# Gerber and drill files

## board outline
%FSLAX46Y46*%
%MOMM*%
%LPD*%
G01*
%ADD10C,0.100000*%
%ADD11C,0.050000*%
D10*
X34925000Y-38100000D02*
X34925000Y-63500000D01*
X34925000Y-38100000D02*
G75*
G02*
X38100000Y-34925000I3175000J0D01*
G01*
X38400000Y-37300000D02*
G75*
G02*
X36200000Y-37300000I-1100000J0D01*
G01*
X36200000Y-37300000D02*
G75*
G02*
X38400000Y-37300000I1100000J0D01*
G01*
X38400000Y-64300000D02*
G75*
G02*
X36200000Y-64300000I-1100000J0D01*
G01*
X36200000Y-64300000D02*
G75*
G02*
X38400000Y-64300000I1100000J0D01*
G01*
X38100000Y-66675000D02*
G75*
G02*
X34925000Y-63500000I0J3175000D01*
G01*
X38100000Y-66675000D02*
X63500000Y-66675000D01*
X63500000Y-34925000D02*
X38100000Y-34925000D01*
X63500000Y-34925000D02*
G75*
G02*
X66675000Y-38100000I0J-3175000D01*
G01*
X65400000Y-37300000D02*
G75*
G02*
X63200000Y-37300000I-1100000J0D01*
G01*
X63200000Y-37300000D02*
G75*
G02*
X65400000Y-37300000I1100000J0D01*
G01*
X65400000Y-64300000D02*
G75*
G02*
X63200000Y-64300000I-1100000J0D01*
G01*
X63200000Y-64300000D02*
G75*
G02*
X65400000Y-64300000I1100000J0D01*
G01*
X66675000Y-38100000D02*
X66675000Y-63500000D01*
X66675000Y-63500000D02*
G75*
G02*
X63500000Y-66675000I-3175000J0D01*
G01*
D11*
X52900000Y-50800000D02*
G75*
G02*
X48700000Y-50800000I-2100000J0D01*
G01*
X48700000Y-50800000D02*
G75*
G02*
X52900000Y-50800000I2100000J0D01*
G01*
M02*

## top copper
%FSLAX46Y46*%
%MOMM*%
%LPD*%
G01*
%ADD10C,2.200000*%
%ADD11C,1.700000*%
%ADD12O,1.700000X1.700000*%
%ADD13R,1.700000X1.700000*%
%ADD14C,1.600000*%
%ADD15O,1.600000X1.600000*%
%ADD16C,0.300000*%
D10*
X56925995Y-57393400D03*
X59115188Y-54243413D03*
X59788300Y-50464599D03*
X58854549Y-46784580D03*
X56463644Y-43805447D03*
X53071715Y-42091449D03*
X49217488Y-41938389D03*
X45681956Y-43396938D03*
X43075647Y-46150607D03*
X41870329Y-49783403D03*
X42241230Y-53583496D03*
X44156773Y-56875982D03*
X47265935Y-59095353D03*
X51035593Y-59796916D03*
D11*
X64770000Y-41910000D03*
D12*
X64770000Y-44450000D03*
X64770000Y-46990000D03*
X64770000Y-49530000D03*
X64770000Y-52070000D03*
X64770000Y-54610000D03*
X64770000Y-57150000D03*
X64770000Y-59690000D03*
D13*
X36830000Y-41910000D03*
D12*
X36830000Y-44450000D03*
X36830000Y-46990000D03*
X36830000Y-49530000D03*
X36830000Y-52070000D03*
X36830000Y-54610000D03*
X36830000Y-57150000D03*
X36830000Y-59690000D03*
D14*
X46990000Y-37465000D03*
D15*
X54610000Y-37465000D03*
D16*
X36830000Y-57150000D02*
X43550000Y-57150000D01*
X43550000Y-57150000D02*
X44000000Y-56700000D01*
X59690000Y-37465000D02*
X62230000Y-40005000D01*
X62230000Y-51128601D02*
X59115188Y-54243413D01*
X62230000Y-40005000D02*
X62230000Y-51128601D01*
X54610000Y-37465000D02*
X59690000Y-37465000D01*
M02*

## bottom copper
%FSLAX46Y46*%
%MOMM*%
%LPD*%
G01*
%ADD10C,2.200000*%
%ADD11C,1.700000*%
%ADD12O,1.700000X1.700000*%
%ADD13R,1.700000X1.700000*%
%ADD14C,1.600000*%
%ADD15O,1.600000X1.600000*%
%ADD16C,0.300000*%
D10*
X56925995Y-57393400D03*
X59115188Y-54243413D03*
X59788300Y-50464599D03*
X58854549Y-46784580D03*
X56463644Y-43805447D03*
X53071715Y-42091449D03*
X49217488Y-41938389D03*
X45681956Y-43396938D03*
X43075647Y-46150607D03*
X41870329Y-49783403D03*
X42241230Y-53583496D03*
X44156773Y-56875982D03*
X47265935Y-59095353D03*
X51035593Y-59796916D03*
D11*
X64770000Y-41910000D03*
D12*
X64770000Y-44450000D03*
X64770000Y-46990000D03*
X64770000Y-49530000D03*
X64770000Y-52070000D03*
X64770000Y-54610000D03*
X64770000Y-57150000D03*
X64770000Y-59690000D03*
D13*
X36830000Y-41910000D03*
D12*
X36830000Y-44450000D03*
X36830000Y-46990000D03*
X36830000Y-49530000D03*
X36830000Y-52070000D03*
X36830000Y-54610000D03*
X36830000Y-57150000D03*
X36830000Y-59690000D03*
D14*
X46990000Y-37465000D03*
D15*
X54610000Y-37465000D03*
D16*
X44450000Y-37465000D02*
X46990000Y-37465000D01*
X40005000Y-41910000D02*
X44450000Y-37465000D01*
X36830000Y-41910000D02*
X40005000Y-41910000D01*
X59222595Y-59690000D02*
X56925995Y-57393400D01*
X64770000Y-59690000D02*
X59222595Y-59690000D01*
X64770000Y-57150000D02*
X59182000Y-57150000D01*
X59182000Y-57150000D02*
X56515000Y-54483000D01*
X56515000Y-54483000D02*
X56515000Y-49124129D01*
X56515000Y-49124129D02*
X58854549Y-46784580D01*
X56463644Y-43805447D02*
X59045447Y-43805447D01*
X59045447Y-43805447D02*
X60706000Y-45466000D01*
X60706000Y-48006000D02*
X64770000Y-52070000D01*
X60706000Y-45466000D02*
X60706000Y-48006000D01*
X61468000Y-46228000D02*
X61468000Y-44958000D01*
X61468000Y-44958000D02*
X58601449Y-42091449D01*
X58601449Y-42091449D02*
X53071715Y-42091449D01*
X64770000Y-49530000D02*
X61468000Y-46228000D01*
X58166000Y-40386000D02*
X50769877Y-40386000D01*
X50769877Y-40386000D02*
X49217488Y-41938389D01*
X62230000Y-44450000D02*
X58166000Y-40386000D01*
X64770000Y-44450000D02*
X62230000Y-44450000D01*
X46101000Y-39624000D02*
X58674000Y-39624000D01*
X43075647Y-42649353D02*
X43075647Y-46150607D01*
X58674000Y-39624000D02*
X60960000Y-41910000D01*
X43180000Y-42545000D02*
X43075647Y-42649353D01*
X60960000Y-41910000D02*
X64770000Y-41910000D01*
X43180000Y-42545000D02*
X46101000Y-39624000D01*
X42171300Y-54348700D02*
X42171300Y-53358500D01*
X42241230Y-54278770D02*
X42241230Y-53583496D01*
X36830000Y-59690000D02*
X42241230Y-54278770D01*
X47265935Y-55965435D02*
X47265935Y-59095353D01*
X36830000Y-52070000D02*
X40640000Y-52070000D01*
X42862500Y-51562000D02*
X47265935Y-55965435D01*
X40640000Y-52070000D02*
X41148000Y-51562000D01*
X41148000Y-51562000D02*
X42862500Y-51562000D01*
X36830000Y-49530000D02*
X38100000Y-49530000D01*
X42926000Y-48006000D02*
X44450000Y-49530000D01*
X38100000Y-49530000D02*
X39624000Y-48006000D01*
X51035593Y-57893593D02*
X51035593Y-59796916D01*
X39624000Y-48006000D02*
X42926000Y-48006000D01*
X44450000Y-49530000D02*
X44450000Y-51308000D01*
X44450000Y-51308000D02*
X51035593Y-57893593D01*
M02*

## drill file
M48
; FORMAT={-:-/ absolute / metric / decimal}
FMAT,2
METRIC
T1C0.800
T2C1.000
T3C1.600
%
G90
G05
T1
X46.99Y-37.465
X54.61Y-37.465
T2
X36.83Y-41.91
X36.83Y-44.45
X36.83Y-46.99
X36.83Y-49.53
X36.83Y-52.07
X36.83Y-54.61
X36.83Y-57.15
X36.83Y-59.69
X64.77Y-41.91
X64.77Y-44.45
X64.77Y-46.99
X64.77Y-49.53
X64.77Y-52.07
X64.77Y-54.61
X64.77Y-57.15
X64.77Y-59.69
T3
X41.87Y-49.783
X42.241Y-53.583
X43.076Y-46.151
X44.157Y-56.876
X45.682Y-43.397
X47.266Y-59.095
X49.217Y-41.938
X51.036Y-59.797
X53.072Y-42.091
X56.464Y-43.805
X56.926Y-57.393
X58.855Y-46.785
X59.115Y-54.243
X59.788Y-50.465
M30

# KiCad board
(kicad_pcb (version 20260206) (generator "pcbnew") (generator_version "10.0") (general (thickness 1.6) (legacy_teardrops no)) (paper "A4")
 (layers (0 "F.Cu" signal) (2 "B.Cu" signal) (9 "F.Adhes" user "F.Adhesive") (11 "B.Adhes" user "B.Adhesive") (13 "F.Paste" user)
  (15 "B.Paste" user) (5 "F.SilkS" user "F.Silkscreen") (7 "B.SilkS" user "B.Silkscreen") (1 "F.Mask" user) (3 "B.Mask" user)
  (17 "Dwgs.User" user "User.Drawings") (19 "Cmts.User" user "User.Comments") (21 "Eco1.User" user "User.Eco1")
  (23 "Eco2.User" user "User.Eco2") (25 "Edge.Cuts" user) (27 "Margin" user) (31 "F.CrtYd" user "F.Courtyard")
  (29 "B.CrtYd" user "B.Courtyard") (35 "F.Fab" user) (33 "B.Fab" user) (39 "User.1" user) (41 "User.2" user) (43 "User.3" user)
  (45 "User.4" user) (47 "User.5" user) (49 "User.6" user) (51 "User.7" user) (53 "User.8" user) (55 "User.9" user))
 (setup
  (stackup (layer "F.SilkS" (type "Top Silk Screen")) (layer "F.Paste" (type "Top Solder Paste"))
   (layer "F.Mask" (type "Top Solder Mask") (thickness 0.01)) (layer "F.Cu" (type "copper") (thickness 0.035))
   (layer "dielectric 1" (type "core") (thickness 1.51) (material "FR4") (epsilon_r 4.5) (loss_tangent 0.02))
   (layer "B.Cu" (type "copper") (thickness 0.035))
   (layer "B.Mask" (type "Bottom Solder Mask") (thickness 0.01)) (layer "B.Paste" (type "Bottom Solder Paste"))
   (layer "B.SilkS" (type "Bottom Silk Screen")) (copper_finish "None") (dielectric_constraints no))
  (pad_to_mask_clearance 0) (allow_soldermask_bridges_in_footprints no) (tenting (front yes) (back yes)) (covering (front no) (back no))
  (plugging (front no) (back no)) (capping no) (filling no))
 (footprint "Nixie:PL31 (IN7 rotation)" (layer "F.Cu") (at 50.8 50.8)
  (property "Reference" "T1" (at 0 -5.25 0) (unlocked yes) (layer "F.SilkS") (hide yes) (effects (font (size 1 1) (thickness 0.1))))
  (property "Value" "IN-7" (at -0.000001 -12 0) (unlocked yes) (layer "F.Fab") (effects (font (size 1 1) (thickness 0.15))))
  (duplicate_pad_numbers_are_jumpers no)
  (fp_circle (center 0 0) (end 2.1 0) (stroke (width 0.05) (type default)) (fill no) (layer "Edge.Cuts"))
  (pad "1" thru_hole circle (at 6.125995 6.5934 181.5) (size 2.2 2.2) (drill 1.6) (layers "*.Cu" "*.Mask") (remove_unused_layers no)
   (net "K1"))
  (pad "2" thru_hole circle (at 8.315188 3.443413 181.5) (size 2.2 2.2) (drill 1.6) (layers "*.Cu" "*.Mask") (remove_unused_layers no)
   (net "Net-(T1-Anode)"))
  (pad "3" thru_hole circle (at 8.9883 -0.335401 181.5) (size 2.2 2.2) (drill 1.6) (layers "*.Cu" "*.Mask") (remove_unused_layers no)
   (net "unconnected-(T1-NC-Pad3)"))
  (pad "4" thru_hole circle (at 8.054549 -4.01542 181.5) (size 2.2 2.2) (drill 1.6) (layers "*.Cu" "*.Mask") (remove_unused_layers no)
   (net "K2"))
  (pad "5" thru_hole circle (at 5.663644 -6.994553 181.5) (size 2.2 2.2) (drill 1.6) (layers "*.Cu" "*.Mask") (remove_unused_layers no)
   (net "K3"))
  (pad "6" thru_hole circle (at 2.271715 -8.708551 181.5) (size 2.2 2.2) (drill 1.6) (layers "*.Cu" "*.Mask") (remove_unused_layers no)
   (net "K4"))
  (pad "7" thru_hole circle (at -1.582512 -8.861611 181.5) (size 2.2 2.2) (drill 1.6) (layers "*.Cu" "*.Mask") (remove_unused_layers no)
   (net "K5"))
  (pad "8" thru_hole circle (at -5.118044 -7.403062 181.5) (size 2.2 2.2) (drill 1.6) (layers "*.Cu" "*.Mask") (remove_unused_layers no)
   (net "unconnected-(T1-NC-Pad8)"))
  (pad "9" thru_hole circle (at -7.724353 -4.649393 181.5) (size 2.2 2.2) (drill 1.6) (layers "*.Cu" "*.Mask") (remove_unused_layers no)
   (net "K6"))
  (pad "10" thru_hole circle (at -8.929671 -1.016597 181.5) (size 2.2 2.2) (drill 1.6) (layers "*.Cu" "*.Mask") (remove_unused_layers no)
   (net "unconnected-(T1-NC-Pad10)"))
  (pad "11" thru_hole circle (at -8.55877 2.783496 181.5) (size 2.2 2.2) (drill 1.6) (layers "*.Cu" "*.Mask") (remove_unused_layers no)
   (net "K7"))
  (pad "12" thru_hole circle (at -6.643227 6.075982 181.5) (size 2.2 2.2) (drill 1.6) (layers "*.Cu" "*.Mask") (remove_unused_layers no)
   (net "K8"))
  (pad "13" thru_hole circle (at -3.534065 8.295353 181.5) (size 2.2 2.2) (drill 1.6) (layers "*.Cu" "*.Mask") (remove_unused_layers no)
   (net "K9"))
  (pad "14" thru_hole circle (at 0.235593 8.996916 181.5) (size 2.2 2.2) (drill 1.6) (layers "*.Cu" "*.Mask") (remove_unused_layers no)
   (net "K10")))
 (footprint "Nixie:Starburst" (layer "F.Cu") (at 43 63.25)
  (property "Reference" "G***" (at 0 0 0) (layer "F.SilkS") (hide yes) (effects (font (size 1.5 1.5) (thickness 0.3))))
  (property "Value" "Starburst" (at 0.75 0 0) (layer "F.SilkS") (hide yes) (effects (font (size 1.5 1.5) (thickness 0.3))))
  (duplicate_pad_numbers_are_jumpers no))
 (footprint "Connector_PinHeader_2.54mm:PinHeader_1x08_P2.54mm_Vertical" (layer "B.Cu") (at 64.77 41.91 180)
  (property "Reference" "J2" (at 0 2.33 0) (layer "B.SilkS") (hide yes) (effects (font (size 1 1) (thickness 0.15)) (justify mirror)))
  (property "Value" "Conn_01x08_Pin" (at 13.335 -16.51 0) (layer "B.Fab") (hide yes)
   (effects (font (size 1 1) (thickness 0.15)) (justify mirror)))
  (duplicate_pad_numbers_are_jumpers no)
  (pad "1" thru_hole circle (at 0 0 180) (size 1.7 1.7) (drill 1) (layers "*.Cu" "*.Mask") (remove_unused_layers no) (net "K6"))
  (pad "2" thru_hole oval (at 0 -2.54 180) (size 1.7 1.7) (drill 1) (layers "*.Cu" "*.Mask") (remove_unused_layers no) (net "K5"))
  (pad "3" thru_hole oval (at 0 -5.08 180) (size 1.7 1.7) (drill 1) (layers "*.Cu" "*.Mask") (remove_unused_layers no)
   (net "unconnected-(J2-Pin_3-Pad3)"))
  (pad "4" thru_hole oval (at 0 -7.62 180) (size 1.7 1.7) (drill 1) (layers "*.Cu" "*.Mask") (remove_unused_layers no) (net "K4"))
  (pad "5" thru_hole oval (at 0 -10.16 180) (size 1.7 1.7) (drill 1) (layers "*.Cu" "*.Mask") (remove_unused_layers no) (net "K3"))
  (pad "6" thru_hole oval (at 0 -12.7 180) (size 1.7 1.7) (drill 1) (layers "*.Cu" "*.Mask") (remove_unused_layers no)
   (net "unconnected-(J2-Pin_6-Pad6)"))
  (pad "7" thru_hole oval (at 0 -15.24 180) (size 1.7 1.7) (drill 1) (layers "*.Cu" "*.Mask") (remove_unused_layers no) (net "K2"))
  (pad "8" thru_hole oval (at 0 -17.78 180) (size 1.7 1.7) (drill 1) (layers "*.Cu" "*.Mask") (remove_unused_layers no) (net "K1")))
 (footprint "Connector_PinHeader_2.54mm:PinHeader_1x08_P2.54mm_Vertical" (layer "B.Cu") (at 36.83 41.91 180)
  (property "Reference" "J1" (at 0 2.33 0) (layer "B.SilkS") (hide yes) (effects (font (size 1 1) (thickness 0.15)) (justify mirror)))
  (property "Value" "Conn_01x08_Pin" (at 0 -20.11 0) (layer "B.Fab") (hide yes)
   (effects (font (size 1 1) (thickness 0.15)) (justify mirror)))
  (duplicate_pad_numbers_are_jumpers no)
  (pad "1" thru_hole rect (at 0 0 180) (size 1.7 1.7) (drill 1) (layers "*.Cu" "*.Mask") (remove_unused_layers no) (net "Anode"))
  (pad "2" thru_hole oval (at 0 -2.54 180) (size 1.7 1.7) (drill 1) (layers "*.Cu" "*.Mask") (remove_unused_layers no)
   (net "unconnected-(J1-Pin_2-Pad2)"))
  (pad "3" thru_hole oval (at 0 -5.08 180) (size 1.7 1.7) (drill 1) (layers "*.Cu" "*.Mask") (remove_unused_layers no)
   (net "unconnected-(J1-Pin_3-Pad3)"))
  (pad "4" thru_hole oval (at 0 -7.62 180) (size 1.7 1.7) (drill 1) (layers "*.Cu" "*.Mask") (remove_unused_layers no) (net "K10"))
  (pad "5" thru_hole oval (at 0 -10.16 180) (size 1.7 1.7) (drill 1) (layers "*.Cu" "*.Mask") (remove_unused_layers no) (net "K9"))
  (pad "6" thru_hole oval (at 0 -12.7 180) (size 1.7 1.7) (drill 1) (layers "*.Cu" "*.Mask") (remove_unused_layers no)
   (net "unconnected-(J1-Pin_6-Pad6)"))
  (pad "7" thru_hole oval (at 0 -15.24 180) (size 1.7 1.7) (drill 1) (layers "*.Cu" "*.Mask") (remove_unused_layers no) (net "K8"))
  (pad "8" thru_hole oval (at 0 -17.78 180) (size 1.7 1.7) (drill 1) (layers "*.Cu" "*.Mask") (remove_unused_layers no) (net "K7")))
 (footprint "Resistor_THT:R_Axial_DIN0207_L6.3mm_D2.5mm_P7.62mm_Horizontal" (layer "B.Cu") (at 46.99 37.465)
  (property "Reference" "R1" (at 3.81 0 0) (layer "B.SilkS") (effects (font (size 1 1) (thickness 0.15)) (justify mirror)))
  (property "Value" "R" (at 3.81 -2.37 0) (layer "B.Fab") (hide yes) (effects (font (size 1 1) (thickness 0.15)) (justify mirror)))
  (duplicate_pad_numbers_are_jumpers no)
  (pad "1" thru_hole circle (at 0 0) (size 1.6 1.6) (drill 0.8) (layers "*.Cu" "*.Mask") (remove_unused_layers no) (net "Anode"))
  (pad "2" thru_hole oval (at 7.62 0) (size 1.6 1.6) (drill 0.8) (layers "*.Cu" "*.Mask") (remove_unused_layers no) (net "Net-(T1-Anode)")))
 (gr_line (start 34.925 38.1) (end 34.925 63.5) (stroke (width 0.1) (type default)) (layer "Edge.Cuts"))
 (gr_arc (start 34.925 38.1) (mid 35.854936 35.854936) (end 38.1 34.925) (stroke (width 0.1) (type default)) (layer "Edge.Cuts"))
 (gr_circle (center 37.3 37.3) (end 38.4 37.3) (stroke (width 0.1) (type default)) (fill no) (layer "Edge.Cuts"))
 (gr_circle (center 37.3 64.3) (end 38.4 64.3) (stroke (width 0.1) (type default)) (fill no) (layer "Edge.Cuts"))
 (gr_arc (start 38.1 66.675) (mid 35.854936 65.745064) (end 34.925 63.5) (stroke (width 0.1) (type default)) (layer "Edge.Cuts"))
 (gr_line (start 38.1 66.675) (end 63.5 66.675) (stroke (width 0.1) (type default)) (layer "Edge.Cuts"))
 (gr_line (start 63.5 34.925) (end 38.1 34.925) (stroke (width 0.1) (type default)) (layer "Edge.Cuts"))
 (gr_arc (start 63.5 34.925) (mid 65.745064 35.854936) (end 66.675 38.1) (stroke (width 0.1) (type default)) (layer "Edge.Cuts"))
 (gr_circle (center 64.3 37.3) (end 65.4 37.3) (stroke (width 0.1) (type default)) (fill no) (layer "Edge.Cuts"))
 (gr_circle (center 64.3 64.3) (end 65.4 64.3) (stroke (width 0.1) (type default)) (fill no) (layer "Edge.Cuts"))
 (gr_line (start 66.675 38.1) (end 66.675 63.5) (stroke (width 0.1) (type default)) (layer "Edge.Cuts"))
 (gr_arc (start 66.675 63.5) (mid 65.745064 65.745064) (end 63.5 66.675) (stroke (width 0.1) (type default)) (layer "Edge.Cuts"))
 (segment (start 44.45 37.465) (end 46.99 37.465) (width 0.3) (layer "B.Cu") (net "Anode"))
 (segment (start 40.005 41.91) (end 44.45 37.465) (width 0.3) (layer "B.Cu") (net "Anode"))
 (segment (start 36.83 41.91) (end 40.005 41.91) (width 0.3) (layer "B.Cu") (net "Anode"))
 (segment (start 59.222595 59.69) (end 56.925995 57.3934) (width 0.3) (layer "B.Cu") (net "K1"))
 (segment (start 64.77 59.69) (end 59.222595 59.69) (width 0.3) (layer "B.Cu") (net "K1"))
 (segment (start 64.77 57.15) (end 59.182 57.15) (width 0.3) (layer "B.Cu") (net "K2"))
 (segment (start 59.182 57.15) (end 56.515 54.483) (width 0.3) (layer "B.Cu") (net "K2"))
 (segment (start 56.515 54.483) (end 56.515 49.124129) (width 0.3) (layer "B.Cu") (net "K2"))
 (segment (start 56.515 49.124129) (end 58.854549 46.78458) (width 0.3) (layer "B.Cu") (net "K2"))
 (segment (start 56.463644 43.805447) (end 59.045447 43.805447) (width 0.3) (layer "B.Cu") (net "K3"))
 (segment (start 59.045447 43.805447) (end 60.706 45.466) (width 0.3) (layer "B.Cu") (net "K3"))
 (segment (start 60.706 48.006) (end 64.77 52.07) (width 0.3) (layer "B.Cu") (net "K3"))
 (segment (start 60.706 45.466) (end 60.706 48.006) (width 0.3) (layer "B.Cu") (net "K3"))
 (segment (start 61.468 46.228) (end 61.468 44.958) (width 0.3) (layer "B.Cu") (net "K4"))
 (segment (start 61.468 44.958) (end 58.601449 42.091449) (width 0.3) (layer "B.Cu") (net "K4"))
 (segment (start 58.601449 42.091449) (end 53.071715 42.091449) (width 0.3) (layer "B.Cu") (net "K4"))
 (segment (start 64.77 49.53) (end 61.468 46.228) (width 0.3) (layer "B.Cu") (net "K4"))
 (segment (start 58.166 40.386) (end 50.769877 40.386) (width 0.3) (layer "B.Cu") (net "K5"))
 (segment (start 50.769877 40.386) (end 49.217488 41.938389) (width 0.3) (layer "B.Cu") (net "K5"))
 (segment (start 62.23 44.45) (end 58.166 40.386) (width 0.3) (layer "B.Cu") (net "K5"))
 (segment (start 64.77 44.45) (end 62.23 44.45) (width 0.3) (layer "B.Cu") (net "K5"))
 (segment (start 46.101 39.624) (end 58.674 39.624) (width 0.3) (layer "B.Cu") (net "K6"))
 (segment (start 43.075647 42.649353) (end 43.075647 46.150607) (width 0.3) (layer "B.Cu") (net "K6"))
 (segment (start 58.674 39.624) (end 60.96 41.91) (width 0.3) (layer "B.Cu") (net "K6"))
 (segment (start 43.18 42.545) (end 43.075647 42.649353) (width 0.3) (layer "B.Cu") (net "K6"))
 (segment (start 60.96 41.91) (end 64.77 41.91) (width 0.3) (layer "B.Cu") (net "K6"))
 (segment (start 43.18 42.545) (end 46.101 39.624) (width 0.3) (layer "B.Cu") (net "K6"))
 (segment (start 42.1713 54.3487) (end 42.1713 53.3585) (width 0.3) (layer "B.Cu") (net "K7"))
 (segment (start 42.24123 54.27877) (end 42.24123 53.583496) (width 0.3) (layer "B.Cu") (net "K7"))
 (segment (start 36.83 59.69) (end 42.24123 54.27877) (width 0.3) (layer "B.Cu") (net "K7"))
 (segment (start 36.83 57.15) (end 43.55 57.15) (width 0.3) (layer "F.Cu") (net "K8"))
 (segment (start 43.55 57.15) (end 44 56.7) (width 0.3) (layer "F.Cu") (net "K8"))
 (segment (start 47.265935 55.965435) (end 47.265935 59.095353) (width 0.3) (layer "B.Cu") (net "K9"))
 (segment (start 36.83 52.07) (end 40.64 52.07) (width 0.3) (layer "B.Cu") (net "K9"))
 (segment (start 42.8625 51.562) (end 47.265935 55.965435) (width 0.3) (layer "B.Cu") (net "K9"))
 (segment (start 40.64 52.07) (end 41.148 51.562) (width 0.3) (layer "B.Cu") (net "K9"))
 (segment (start 41.148 51.562) (end 42.8625 51.562) (width 0.3) (layer "B.Cu") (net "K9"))
 (segment (start 36.83 49.53) (end 38.1 49.53) (width 0.3) (layer "B.Cu") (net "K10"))
 (segment (start 42.926 48.006) (end 44.45 49.53) (width 0.3) (layer "B.Cu") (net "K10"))
 (segment (start 38.1 49.53) (end 39.624 48.006) (width 0.3) (layer "B.Cu") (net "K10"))
 (segment (start 51.035593 57.893593) (end 51.035593 59.796916) (width 0.3) (layer "B.Cu") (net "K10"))
 (segment (start 39.624 48.006) (end 42.926 48.006) (width 0.3) (layer "B.Cu") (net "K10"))
 (segment (start 44.45 49.53) (end 44.45 51.308) (width 0.3) (layer "B.Cu") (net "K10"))
 (segment (start 44.45 51.308) (end 51.035593 57.893593) (width 0.3) (layer "B.Cu") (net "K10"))
 (segment (start 59.69 37.465) (end 62.23 40.005) (width 0.3) (layer "F.Cu") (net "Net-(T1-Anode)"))
 (segment (start 62.23 51.128601) (end 59.115188 54.243413) (width 0.3) (layer "F.Cu") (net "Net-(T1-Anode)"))
 (segment (start 62.23 40.005) (end 62.23 51.128601) (width 0.3) (layer "F.Cu") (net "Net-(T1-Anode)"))
 (segment (start 54.61 37.465) (end 59.69 37.465) (width 0.3) (layer "F.Cu") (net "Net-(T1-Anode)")))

